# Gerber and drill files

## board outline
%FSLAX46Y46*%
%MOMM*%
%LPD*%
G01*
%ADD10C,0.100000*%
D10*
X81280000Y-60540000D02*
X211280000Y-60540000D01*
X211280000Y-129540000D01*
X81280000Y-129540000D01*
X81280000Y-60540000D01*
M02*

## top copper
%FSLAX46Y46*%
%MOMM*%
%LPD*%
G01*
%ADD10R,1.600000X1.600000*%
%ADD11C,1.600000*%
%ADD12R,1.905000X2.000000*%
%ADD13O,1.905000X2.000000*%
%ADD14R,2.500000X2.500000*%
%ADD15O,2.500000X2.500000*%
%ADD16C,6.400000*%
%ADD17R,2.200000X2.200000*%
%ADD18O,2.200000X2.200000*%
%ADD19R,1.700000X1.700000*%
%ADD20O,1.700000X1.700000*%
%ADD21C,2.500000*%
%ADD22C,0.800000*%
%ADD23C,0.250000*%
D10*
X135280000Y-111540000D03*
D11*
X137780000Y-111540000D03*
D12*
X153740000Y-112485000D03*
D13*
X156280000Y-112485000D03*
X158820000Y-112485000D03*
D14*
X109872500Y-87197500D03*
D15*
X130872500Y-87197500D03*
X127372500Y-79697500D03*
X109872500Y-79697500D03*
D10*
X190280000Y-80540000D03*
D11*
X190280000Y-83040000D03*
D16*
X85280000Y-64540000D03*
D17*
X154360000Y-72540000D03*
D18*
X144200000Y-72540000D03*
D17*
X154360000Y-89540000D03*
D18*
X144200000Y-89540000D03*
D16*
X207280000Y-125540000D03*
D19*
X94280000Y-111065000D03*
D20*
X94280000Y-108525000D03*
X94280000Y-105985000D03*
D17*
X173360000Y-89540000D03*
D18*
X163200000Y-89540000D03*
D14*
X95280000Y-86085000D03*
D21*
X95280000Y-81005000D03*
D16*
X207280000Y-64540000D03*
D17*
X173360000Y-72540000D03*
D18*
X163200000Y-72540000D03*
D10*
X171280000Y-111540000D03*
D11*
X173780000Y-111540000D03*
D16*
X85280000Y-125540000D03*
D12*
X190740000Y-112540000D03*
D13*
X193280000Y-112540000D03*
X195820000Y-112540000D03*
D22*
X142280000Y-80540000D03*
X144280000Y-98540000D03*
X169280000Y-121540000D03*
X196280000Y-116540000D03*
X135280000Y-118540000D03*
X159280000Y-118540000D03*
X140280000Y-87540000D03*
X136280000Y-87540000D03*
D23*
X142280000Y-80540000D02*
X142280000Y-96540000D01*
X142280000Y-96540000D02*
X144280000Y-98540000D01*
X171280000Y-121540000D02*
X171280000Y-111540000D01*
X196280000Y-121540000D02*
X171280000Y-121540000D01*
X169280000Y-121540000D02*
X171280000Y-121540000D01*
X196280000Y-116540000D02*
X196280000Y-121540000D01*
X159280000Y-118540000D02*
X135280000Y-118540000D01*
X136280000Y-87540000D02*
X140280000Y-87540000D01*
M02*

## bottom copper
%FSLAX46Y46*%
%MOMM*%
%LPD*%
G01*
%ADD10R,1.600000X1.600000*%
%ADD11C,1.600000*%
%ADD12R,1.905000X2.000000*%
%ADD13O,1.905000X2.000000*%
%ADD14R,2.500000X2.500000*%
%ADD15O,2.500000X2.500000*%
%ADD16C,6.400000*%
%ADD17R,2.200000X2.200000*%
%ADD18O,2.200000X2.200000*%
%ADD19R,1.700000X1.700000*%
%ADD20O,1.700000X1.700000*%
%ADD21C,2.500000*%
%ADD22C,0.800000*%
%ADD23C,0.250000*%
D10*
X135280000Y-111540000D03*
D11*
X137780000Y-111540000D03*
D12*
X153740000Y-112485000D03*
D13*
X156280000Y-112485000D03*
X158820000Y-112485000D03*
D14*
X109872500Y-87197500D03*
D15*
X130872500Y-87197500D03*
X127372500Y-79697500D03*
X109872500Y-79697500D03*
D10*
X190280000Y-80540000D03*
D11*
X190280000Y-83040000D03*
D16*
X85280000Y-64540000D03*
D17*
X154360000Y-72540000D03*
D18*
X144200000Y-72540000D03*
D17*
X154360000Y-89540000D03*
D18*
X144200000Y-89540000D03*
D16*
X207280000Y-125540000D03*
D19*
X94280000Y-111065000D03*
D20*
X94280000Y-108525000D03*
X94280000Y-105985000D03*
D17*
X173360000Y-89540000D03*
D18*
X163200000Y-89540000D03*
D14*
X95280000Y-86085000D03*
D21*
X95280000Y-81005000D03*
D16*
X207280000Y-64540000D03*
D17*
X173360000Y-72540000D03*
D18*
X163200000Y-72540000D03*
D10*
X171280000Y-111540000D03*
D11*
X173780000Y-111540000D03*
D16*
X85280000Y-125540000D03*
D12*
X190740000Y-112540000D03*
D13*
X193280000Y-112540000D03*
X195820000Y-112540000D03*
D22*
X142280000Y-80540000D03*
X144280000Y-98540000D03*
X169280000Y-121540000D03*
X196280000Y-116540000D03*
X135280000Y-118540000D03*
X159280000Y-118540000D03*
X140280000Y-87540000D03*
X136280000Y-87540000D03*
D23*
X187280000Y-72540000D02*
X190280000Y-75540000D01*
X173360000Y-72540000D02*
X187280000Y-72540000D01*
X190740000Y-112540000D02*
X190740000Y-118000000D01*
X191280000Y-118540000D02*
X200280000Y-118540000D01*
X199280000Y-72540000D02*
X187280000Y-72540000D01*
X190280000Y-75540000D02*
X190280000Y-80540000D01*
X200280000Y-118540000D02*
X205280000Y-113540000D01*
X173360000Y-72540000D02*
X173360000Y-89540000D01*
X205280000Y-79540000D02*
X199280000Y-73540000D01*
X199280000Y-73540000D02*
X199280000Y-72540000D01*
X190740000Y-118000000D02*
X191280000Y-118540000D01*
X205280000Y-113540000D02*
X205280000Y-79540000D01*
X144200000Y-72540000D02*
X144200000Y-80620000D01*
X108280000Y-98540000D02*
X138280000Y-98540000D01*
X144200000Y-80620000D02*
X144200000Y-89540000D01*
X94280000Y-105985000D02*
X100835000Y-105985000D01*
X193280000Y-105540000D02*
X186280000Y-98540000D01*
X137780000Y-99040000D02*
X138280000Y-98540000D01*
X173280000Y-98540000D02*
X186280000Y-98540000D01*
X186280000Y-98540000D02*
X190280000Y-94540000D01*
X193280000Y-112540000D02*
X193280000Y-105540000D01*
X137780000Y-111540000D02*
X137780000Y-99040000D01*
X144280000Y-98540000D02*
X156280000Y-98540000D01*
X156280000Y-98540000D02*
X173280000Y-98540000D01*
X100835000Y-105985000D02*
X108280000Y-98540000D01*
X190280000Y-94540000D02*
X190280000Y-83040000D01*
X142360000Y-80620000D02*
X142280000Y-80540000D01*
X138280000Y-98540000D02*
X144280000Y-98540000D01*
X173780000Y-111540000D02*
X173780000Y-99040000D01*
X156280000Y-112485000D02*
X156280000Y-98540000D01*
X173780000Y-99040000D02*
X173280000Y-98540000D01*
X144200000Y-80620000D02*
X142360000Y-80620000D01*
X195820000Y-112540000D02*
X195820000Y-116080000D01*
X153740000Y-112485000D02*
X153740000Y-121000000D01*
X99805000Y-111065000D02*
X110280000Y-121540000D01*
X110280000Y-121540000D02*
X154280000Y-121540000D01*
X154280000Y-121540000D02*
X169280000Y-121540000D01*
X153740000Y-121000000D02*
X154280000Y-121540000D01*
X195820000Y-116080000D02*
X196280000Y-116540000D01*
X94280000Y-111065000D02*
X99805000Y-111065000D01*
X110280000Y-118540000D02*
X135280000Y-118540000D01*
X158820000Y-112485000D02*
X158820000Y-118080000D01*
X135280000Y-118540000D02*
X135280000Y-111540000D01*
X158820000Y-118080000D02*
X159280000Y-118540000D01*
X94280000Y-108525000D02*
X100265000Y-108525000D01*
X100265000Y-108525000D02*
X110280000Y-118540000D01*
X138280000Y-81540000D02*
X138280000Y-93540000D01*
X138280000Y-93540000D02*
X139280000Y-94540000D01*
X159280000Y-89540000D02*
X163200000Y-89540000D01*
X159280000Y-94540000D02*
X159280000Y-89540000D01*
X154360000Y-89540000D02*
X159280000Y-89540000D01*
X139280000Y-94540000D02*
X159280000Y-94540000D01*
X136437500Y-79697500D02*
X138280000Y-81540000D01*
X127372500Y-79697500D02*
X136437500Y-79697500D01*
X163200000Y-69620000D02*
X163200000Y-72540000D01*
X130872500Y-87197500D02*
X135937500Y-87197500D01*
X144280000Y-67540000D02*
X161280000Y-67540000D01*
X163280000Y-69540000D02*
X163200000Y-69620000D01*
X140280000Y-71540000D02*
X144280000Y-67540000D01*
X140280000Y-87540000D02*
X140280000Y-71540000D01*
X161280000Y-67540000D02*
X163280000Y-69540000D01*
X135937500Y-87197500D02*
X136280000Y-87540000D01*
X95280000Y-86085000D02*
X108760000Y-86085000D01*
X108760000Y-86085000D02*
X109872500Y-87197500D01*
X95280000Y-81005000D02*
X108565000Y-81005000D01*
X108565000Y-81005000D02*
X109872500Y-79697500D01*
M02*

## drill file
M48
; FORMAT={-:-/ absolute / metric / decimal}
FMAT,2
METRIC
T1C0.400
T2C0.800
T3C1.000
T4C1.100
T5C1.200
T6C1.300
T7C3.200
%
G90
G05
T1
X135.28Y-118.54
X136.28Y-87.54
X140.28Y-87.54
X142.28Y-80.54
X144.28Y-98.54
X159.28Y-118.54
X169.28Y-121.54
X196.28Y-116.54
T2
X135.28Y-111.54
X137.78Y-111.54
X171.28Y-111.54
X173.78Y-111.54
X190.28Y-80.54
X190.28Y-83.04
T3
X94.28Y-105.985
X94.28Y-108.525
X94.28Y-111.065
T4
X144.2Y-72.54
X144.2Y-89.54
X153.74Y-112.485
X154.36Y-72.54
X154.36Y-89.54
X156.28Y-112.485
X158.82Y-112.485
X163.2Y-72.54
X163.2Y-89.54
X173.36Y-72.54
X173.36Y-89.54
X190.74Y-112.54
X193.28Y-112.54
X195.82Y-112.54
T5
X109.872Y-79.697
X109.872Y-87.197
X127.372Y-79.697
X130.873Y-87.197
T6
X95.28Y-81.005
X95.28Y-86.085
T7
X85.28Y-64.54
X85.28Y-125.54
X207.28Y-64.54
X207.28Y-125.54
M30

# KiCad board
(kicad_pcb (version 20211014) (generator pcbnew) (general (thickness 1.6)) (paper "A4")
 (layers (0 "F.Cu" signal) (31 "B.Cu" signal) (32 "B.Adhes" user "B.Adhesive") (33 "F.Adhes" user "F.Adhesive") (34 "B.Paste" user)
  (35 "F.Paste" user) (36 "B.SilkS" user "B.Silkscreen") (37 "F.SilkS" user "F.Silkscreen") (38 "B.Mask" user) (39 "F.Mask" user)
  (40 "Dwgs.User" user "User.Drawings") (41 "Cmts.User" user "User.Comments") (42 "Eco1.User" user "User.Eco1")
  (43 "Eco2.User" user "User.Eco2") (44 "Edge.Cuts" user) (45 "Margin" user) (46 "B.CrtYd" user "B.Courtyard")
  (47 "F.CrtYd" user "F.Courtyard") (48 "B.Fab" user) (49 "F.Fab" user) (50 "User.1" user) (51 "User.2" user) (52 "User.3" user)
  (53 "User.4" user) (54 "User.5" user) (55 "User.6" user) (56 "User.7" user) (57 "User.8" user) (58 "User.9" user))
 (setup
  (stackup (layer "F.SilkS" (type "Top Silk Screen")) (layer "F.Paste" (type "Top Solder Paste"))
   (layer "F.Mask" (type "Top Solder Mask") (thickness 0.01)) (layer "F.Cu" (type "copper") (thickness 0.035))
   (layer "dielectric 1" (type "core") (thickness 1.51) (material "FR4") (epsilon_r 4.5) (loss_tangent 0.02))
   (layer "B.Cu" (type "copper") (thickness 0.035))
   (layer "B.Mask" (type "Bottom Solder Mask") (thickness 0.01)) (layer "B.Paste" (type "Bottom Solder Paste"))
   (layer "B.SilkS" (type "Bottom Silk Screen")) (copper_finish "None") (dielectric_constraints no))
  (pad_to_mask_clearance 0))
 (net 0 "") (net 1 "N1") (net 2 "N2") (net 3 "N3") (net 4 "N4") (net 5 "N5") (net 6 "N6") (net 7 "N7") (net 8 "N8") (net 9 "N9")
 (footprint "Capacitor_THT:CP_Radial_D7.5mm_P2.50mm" (layer "F.Cu") (at 135.28 111.54)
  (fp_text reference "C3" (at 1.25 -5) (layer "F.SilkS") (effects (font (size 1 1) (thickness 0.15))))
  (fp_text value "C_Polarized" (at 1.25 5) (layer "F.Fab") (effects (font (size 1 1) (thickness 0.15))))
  (pad "1" thru_hole rect (at 0 0) (size 1.6 1.6) (drill 0.8) (layers *.Cu *.Mask) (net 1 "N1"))
  (pad "2" thru_hole circle (at 2.5 0) (size 1.6 1.6) (drill 0.8) (layers *.Cu *.Mask) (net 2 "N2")))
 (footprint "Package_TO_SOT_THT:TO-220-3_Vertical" (layer "F.Cu") (at 153.74 112.485)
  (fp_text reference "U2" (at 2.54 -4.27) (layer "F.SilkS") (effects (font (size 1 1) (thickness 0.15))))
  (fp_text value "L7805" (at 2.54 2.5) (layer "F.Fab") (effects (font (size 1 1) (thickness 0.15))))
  (pad "1" thru_hole rect (at 0 0) (size 1.905 2) (drill 1.1) (layers *.Cu *.Mask) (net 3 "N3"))
  (pad "2" thru_hole oval (at 2.54 0) (size 1.905 2) (drill 1.1) (layers *.Cu *.Mask) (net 2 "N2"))
  (pad "3" thru_hole oval (at 5.08 0) (size 1.905 2) (drill 1.1) (layers *.Cu *.Mask) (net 1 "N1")))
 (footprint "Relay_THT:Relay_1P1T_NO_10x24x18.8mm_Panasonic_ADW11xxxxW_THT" (layer "F.Cu") (at 109.8725 87.1975 90)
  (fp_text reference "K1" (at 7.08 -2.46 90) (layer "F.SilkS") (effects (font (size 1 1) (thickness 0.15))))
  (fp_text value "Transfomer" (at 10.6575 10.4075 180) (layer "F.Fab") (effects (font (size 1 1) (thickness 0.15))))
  (pad "1" thru_hole rect (at 0 0 90) (size 2.5 2.5) (drill 1.2) (layers *.Cu *.Mask) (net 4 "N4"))
  (pad "3" thru_hole oval (at 0 21 90) (size 2.5 2.5) (drill 1.2) (layers *.Cu *.Mask) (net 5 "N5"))
  (pad "5" thru_hole oval (at 7.5 17.5 90) (size 2.5 2.5) (drill 1.2) (layers *.Cu *.Mask) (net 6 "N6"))
  (pad "6" thru_hole oval (at 7.5 0 90) (size 2.5 2.5) (drill 1.2) (layers *.Cu *.Mask) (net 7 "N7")))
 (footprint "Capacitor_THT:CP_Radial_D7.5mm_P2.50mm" (layer "F.Cu") (at 190.28 80.54 -90)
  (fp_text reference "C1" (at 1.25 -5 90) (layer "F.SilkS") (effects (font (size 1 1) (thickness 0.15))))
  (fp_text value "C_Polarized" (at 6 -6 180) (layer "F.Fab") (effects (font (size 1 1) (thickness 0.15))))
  (pad "1" thru_hole rect (at 0 0 270) (size 1.6 1.6) (drill 0.8) (layers *.Cu *.Mask) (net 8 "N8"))
  (pad "2" thru_hole circle (at 2.5 0 270) (size 1.6 1.6) (drill 0.8) (layers *.Cu *.Mask) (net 2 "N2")))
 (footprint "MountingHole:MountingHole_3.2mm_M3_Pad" (layer "F.Cu") (at 85.28 64.54)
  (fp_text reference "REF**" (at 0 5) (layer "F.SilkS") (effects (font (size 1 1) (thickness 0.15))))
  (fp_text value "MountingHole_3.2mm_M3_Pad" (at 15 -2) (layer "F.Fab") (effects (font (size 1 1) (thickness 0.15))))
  (pad "1" thru_hole circle (at 0 0) (size 6.4 6.4) (drill 3.2) (layers *.Cu *.Mask)))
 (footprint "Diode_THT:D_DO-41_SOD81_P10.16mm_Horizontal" (layer "F.Cu") (at 154.36 72.54 180)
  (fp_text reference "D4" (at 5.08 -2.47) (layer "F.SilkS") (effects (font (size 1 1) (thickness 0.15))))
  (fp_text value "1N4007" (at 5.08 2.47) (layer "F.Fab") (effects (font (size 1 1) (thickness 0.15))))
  (pad "1" thru_hole rect (at 0 0 180) (size 2.2 2.2) (drill 1.1) (layers *.Cu *.Mask) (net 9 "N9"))
  (pad "2" thru_hole oval (at 10.16 0 180) (size 2.2 2.2) (drill 1.1) (layers *.Cu *.Mask) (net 2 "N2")))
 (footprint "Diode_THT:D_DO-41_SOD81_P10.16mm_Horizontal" (layer "F.Cu") (at 154.36 89.54 180)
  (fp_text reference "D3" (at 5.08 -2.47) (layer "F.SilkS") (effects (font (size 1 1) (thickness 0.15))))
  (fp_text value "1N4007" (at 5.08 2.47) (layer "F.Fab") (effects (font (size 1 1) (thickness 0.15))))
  (pad "1" thru_hole rect (at 0 0 180) (size 2.2 2.2) (drill 1.1) (layers *.Cu *.Mask) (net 6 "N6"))
  (pad "2" thru_hole oval (at 10.16 0 180) (size 2.2 2.2) (drill 1.1) (layers *.Cu *.Mask) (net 2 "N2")))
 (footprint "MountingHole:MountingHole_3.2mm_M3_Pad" (layer "F.Cu") (at 207.28 125.54)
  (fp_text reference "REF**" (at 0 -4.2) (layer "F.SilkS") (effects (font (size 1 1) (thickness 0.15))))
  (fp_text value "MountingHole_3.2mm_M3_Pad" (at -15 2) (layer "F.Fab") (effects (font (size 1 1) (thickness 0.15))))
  (pad "1" thru_hole circle (at 0 0) (size 6.4 6.4) (drill 3.2) (layers *.Cu *.Mask)))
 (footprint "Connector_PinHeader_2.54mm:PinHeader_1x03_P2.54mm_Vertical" (layer "F.Cu") (at 94.28 111.065 180)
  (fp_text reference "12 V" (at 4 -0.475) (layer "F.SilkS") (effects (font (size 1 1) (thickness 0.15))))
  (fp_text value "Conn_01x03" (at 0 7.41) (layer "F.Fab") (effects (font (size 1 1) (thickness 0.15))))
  (pad "1" thru_hole rect (at 0 0 180) (size 1.7 1.7) (drill 1) (layers *.Cu *.Mask) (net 3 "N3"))
  (pad "2" thru_hole oval (at 0 2.54 180) (size 1.7 1.7) (drill 1) (layers *.Cu *.Mask) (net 1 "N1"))
  (pad "3" thru_hole oval (at 0 5.08 180) (size 1.7 1.7) (drill 1) (layers *.Cu *.Mask) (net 2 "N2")))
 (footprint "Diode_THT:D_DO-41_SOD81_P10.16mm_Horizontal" (layer "F.Cu") (at 173.36 89.54 180)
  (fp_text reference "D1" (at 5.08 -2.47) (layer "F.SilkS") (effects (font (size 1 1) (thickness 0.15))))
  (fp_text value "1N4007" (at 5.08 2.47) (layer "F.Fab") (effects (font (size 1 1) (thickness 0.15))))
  (pad "1" thru_hole rect (at 0 0 180) (size 2.2 2.2) (drill 1.1) (layers *.Cu *.Mask) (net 8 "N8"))
  (pad "2" thru_hole oval (at 10.16 0 180) (size 2.2 2.2) (drill 1.1) (layers *.Cu *.Mask) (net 6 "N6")))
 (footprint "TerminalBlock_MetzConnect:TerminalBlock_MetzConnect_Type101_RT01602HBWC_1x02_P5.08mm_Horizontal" (layer "F.Cu")
  (at 95.28 86.085 90)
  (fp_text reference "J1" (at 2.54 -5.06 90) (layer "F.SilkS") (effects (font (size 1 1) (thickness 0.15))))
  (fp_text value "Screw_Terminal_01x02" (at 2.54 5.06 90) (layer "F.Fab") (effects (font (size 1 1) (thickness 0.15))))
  (pad "1" thru_hole rect (at 0 0 90) (size 2.5 2.5) (drill 1.3) (layers *.Cu *.Mask) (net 4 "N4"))
  (pad "2" thru_hole circle (at 5.08 0 90) (size 2.5 2.5) (drill 1.3) (layers *.Cu *.Mask) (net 7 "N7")))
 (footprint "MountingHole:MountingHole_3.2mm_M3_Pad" (layer "F.Cu") (at 207.28 64.54)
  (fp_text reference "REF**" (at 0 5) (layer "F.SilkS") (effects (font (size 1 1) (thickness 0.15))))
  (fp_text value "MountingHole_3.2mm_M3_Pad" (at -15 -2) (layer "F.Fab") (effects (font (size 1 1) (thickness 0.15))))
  (pad "1" thru_hole circle (at 0 0) (size 6.4 6.4) (drill 3.2) (layers *.Cu *.Mask)))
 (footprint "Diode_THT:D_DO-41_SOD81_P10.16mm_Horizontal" (layer "F.Cu") (at 173.36 72.54 180)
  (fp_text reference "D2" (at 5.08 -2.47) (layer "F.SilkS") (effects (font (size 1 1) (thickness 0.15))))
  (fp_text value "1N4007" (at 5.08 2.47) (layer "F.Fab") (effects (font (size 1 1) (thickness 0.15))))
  (pad "1" thru_hole rect (at 0 0 180) (size 2.2 2.2) (drill 1.1) (layers *.Cu *.Mask) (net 8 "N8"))
  (pad "2" thru_hole oval (at 10.16 0 180) (size 2.2 2.2) (drill 1.1) (layers *.Cu *.Mask) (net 5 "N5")))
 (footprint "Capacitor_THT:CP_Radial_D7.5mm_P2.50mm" (layer "F.Cu") (at 171.28 111.54)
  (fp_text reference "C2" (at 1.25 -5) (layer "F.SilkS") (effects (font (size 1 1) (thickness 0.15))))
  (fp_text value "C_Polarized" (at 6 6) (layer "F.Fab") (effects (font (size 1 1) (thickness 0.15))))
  (pad "1" thru_hole rect (at 0 0) (size 1.6 1.6) (drill 0.8) (layers *.Cu *.Mask) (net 3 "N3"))
  (pad "2" thru_hole circle (at 2.5 0) (size 1.6 1.6) (drill 0.8) (layers *.Cu *.Mask) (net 2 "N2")))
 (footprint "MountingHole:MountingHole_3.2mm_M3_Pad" (layer "F.Cu") (at 85.28 125.54)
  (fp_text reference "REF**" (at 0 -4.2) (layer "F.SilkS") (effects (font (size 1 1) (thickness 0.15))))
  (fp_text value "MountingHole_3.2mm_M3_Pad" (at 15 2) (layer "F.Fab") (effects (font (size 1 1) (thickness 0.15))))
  (pad "1" thru_hole circle (at 0 0) (size 6.4 6.4) (drill 3.2) (layers *.Cu *.Mask)))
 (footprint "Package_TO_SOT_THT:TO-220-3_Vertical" (layer "F.Cu") (at 190.74 112.54)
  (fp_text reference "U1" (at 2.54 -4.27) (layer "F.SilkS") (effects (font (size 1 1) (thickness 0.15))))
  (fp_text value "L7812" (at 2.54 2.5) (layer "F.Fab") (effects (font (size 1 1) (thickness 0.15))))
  (pad "1" thru_hole rect (at 0 0) (size 1.905 2) (drill 1.1) (layers *.Cu *.Mask) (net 8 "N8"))
  (pad "2" thru_hole oval (at 2.54 0) (size 1.905 2) (drill 1.1) (layers *.Cu *.Mask) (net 2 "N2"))
  (pad "3" thru_hole oval (at 5.08 0) (size 1.905 2) (drill 1.1) (layers *.Cu *.Mask) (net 3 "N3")))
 (gr_rect (start 81.28 60.54) (end 211.28 129.54) (layer "Edge.Cuts") (width 0.1) (fill none))
 (segment (start 187.28 72.54) (end 190.28 75.54) (width 0.25) (layer "B.Cu") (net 8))
 (segment (start 173.36 72.54) (end 187.28 72.54) (width 0.25) (layer "B.Cu") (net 8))
 (segment (start 190.74 112.54) (end 190.74 118) (width 0.25) (layer "B.Cu") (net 8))
 (segment (start 191.28 118.54) (end 200.28 118.54) (width 0.25) (layer "B.Cu") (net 8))
 (segment (start 199.28 72.54) (end 187.28 72.54) (width 0.25) (layer "B.Cu") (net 8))
 (segment (start 190.28 75.54) (end 190.28 80.54) (width 0.25) (layer "B.Cu") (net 8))
 (segment (start 200.28 118.54) (end 205.28 113.54) (width 0.25) (layer "B.Cu") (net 8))
 (segment (start 173.36 72.54) (end 173.36 89.54) (width 0.25) (layer "B.Cu") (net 8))
 (segment (start 205.28 79.54) (end 199.28 73.54) (width 0.25) (layer "B.Cu") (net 8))
 (segment (start 199.28 73.54) (end 199.28 72.54) (width 0.25) (layer "B.Cu") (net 8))
 (segment (start 190.74 118) (end 191.28 118.54) (width 0.25) (layer "B.Cu") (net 8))
 (segment (start 205.28 113.54) (end 205.28 79.54) (width 0.25) (layer "B.Cu") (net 8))
 (segment (start 142.28 80.54) (end 142.28 96.54) (width 0.25) (layer "F.Cu") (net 2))
 (segment (start 142.28 96.54) (end 144.28 98.54) (width 0.25) (layer "F.Cu") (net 2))
 (via (at 142.28 80.54) (size 0.8) (drill 0.4) (layers "F.Cu" "B.Cu") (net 2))
 (via (at 144.28 98.54) (size 0.8) (drill 0.4) (layers "F.Cu" "B.Cu") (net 2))
 (segment (start 144.2 72.54) (end 144.2 80.62) (width 0.25) (layer "B.Cu") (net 2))
 (segment (start 108.28 98.54) (end 138.28 98.54) (width 0.25) (layer "B.Cu") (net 2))
 (segment (start 144.2 80.62) (end 144.2 89.54) (width 0.25) (layer "B.Cu") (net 2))
 (segment (start 94.28 105.985) (end 100.835 105.985) (width 0.25) (layer "B.Cu") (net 2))
 (segment (start 193.28 105.54) (end 186.28 98.54) (width 0.25) (layer "B.Cu") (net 2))
 (segment (start 137.78 99.04) (end 138.28 98.54) (width 0.25) (layer "B.Cu") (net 2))
 (segment (start 173.28 98.54) (end 186.28 98.54) (width 0.25) (layer "B.Cu") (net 2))
 (segment (start 186.28 98.54) (end 190.28 94.54) (width 0.25) (layer "B.Cu") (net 2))
 (segment (start 193.28 112.54) (end 193.28 105.54) (width 0.25) (layer "B.Cu") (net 2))
 (segment (start 137.78 111.54) (end 137.78 99.04) (width 0.25) (layer "B.Cu") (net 2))
 (segment (start 144.28 98.54) (end 156.28 98.54) (width 0.25) (layer "B.Cu") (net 2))
 (segment (start 156.28 98.54) (end 173.28 98.54) (width 0.25) (layer "B.Cu") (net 2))
 (segment (start 100.835 105.985) (end 108.28 98.54) (width 0.25) (layer "B.Cu") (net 2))
 (segment (start 190.28 94.54) (end 190.28 83.04) (width 0.25) (layer "B.Cu") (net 2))
 (segment (start 142.36 80.62) (end 142.28 80.54) (width 0.25) (layer "B.Cu") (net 2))
 (segment (start 138.28 98.54) (end 144.28 98.54) (width 0.25) (layer "B.Cu") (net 2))
 (segment (start 173.78 111.54) (end 173.78 99.04) (width 0.25) (layer "B.Cu") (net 2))
 (segment (start 156.28 112.485) (end 156.28 98.54) (width 0.25) (layer "B.Cu") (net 2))
 (segment (start 173.78 99.04) (end 173.28 98.54) (width 0.25) (layer "B.Cu") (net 2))
 (segment (start 144.2 80.62) (end 142.36 80.62) (width 0.25) (layer "B.Cu") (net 2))
 (segment (start 171.28 121.54) (end 171.28 111.54) (width 0.25) (layer "F.Cu") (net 3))
 (segment (start 196.28 121.54) (end 171.28 121.54) (width 0.25) (layer "F.Cu") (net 3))
 (segment (start 169.28 121.54) (end 171.28 121.54) (width 0.25) (layer "F.Cu") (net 3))
 (segment (start 196.28 116.54) (end 196.28 121.54) (width 0.25) (layer "F.Cu") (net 3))
 (via (at 169.28 121.54) (size 0.8) (drill 0.4) (layers "F.Cu" "B.Cu") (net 3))
 (via (at 196.28 116.54) (size 0.8) (drill 0.4) (layers "F.Cu" "B.Cu") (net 3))
 (segment (start 195.82 112.54) (end 195.82 116.08) (width 0.25) (layer "B.Cu") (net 3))
 (segment (start 153.74 112.485) (end 153.74 121) (width 0.25) (layer "B.Cu") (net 3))
 (segment (start 99.805 111.065) (end 110.28 121.54) (width 0.25) (layer "B.Cu") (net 3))
 (segment (start 110.28 121.54) (end 154.28 121.54) (width 0.25) (layer "B.Cu") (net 3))
 (segment (start 154.28 121.54) (end 169.28 121.54) (width 0.25) (layer "B.Cu") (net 3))
 (segment (start 153.74 121) (end 154.28 121.54) (width 0.25) (layer "B.Cu") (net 3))
 (segment (start 195.82 116.08) (end 196.28 116.54) (width 0.25) (layer "B.Cu") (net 3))
 (segment (start 94.28 111.065) (end 99.805 111.065) (width 0.25) (layer "B.Cu") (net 3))
 (segment (start 159.28 118.54) (end 135.28 118.54) (width 0.25) (layer "F.Cu") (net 1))
 (via (at 135.28 118.54) (size 0.8) (drill 0.4) (layers "F.Cu" "B.Cu") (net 1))
 (via (at 159.28 118.54) (size 0.8) (drill 0.4) (layers "F.Cu" "B.Cu") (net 1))
 (segment (start 110.28 118.54) (end 135.28 118.54) (width 0.25) (layer "B.Cu") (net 1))
 (segment (start 158.82 112.485) (end 158.82 118.08) (width 0.25) (layer "B.Cu") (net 1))
 (segment (start 135.28 118.54) (end 135.28 111.54) (width 0.25) (layer "B.Cu") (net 1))
 (segment (start 158.82 118.08) (end 159.28 118.54) (width 0.25) (layer "B.Cu") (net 1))
 (segment (start 94.28 108.525) (end 100.265 108.525) (width 0.25) (layer "B.Cu") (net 1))
 (segment (start 100.265 108.525) (end 110.28 118.54) (width 0.25) (layer "B.Cu") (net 1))
 (segment (start 138.28 81.54) (end 138.28 93.54) (width 0.25) (layer "B.Cu") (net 6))
 (segment (start 138.28 93.54) (end 139.28 94.54) (width 0.25) (layer "B.Cu") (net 6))
 (segment (start 159.28 89.54) (end 163.2 89.54) (width 0.25) (layer "B.Cu") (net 6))
 (segment (start 159.28 94.54) (end 159.28 89.54) (width 0.25) (layer "B.Cu") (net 6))
 (segment (start 154.36 89.54) (end 159.28 89.54) (width 0.25) (layer "B.Cu") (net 6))
 (segment (start 139.28 94.54) (end 159.28 94.54) (width 0.25) (layer "B.Cu") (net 6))
 (segment (start 136.4375 79.6975) (end 138.28 81.54) (width 0.25) (layer "B.Cu") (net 6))
 (segment (start 127.3725 79.6975) (end 136.4375 79.6975) (width 0.25) (layer "B.Cu") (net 6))
 (segment (start 136.28 87.54) (end 140.28 87.54) (width 0.25) (layer "F.Cu") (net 5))
 (via (at 140.28 87.54) (size 0.8) (drill 0.4) (layers "F.Cu" "B.Cu") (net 5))
 (via (at 136.28 87.54) (size 0.8) (drill 0.4) (layers "F.Cu" "B.Cu") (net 5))
 (segment (start 163.2 69.62) (end 163.2 72.54) (width 0.25) (layer "B.Cu") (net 5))
 (segment (start 130.8725 87.1975) (end 135.9375 87.1975) (width 0.25) (layer "B.Cu") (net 5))
 (segment (start 144.28 67.54) (end 161.28 67.54) (width 0.25) (layer "B.Cu") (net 5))
 (segment (start 163.28 69.54) (end 163.2 69.62) (width 0.25) (layer "B.Cu") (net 5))
 (segment (start 140.28 71.54) (end 144.28 67.54) (width 0.25) (layer "B.Cu") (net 5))
 (segment (start 140.28 87.54) (end 140.28 71.54) (width 0.25) (layer "B.Cu") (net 5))
 (segment (start 161.28 67.54) (end 163.28 69.54) (width 0.25) (layer "B.Cu") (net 5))
 (segment (start 135.9375 87.1975) (end 136.28 87.54) (width 0.25) (layer "B.Cu") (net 5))
 (segment (start 95.28 86.085) (end 108.76 86.085) (width 0.25) (layer "B.Cu") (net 4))
 (segment (start 108.76 86.085) (end 109.8725 87.1975) (width 0.25) (layer "B.Cu") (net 4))
 (segment (start 95.28 81.005) (end 108.565 81.005) (width 0.25) (layer "B.Cu") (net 7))
 (segment (start 108.565 81.005) (end 109.8725 79.6975) (width 0.25) (layer "B.Cu") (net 7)))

